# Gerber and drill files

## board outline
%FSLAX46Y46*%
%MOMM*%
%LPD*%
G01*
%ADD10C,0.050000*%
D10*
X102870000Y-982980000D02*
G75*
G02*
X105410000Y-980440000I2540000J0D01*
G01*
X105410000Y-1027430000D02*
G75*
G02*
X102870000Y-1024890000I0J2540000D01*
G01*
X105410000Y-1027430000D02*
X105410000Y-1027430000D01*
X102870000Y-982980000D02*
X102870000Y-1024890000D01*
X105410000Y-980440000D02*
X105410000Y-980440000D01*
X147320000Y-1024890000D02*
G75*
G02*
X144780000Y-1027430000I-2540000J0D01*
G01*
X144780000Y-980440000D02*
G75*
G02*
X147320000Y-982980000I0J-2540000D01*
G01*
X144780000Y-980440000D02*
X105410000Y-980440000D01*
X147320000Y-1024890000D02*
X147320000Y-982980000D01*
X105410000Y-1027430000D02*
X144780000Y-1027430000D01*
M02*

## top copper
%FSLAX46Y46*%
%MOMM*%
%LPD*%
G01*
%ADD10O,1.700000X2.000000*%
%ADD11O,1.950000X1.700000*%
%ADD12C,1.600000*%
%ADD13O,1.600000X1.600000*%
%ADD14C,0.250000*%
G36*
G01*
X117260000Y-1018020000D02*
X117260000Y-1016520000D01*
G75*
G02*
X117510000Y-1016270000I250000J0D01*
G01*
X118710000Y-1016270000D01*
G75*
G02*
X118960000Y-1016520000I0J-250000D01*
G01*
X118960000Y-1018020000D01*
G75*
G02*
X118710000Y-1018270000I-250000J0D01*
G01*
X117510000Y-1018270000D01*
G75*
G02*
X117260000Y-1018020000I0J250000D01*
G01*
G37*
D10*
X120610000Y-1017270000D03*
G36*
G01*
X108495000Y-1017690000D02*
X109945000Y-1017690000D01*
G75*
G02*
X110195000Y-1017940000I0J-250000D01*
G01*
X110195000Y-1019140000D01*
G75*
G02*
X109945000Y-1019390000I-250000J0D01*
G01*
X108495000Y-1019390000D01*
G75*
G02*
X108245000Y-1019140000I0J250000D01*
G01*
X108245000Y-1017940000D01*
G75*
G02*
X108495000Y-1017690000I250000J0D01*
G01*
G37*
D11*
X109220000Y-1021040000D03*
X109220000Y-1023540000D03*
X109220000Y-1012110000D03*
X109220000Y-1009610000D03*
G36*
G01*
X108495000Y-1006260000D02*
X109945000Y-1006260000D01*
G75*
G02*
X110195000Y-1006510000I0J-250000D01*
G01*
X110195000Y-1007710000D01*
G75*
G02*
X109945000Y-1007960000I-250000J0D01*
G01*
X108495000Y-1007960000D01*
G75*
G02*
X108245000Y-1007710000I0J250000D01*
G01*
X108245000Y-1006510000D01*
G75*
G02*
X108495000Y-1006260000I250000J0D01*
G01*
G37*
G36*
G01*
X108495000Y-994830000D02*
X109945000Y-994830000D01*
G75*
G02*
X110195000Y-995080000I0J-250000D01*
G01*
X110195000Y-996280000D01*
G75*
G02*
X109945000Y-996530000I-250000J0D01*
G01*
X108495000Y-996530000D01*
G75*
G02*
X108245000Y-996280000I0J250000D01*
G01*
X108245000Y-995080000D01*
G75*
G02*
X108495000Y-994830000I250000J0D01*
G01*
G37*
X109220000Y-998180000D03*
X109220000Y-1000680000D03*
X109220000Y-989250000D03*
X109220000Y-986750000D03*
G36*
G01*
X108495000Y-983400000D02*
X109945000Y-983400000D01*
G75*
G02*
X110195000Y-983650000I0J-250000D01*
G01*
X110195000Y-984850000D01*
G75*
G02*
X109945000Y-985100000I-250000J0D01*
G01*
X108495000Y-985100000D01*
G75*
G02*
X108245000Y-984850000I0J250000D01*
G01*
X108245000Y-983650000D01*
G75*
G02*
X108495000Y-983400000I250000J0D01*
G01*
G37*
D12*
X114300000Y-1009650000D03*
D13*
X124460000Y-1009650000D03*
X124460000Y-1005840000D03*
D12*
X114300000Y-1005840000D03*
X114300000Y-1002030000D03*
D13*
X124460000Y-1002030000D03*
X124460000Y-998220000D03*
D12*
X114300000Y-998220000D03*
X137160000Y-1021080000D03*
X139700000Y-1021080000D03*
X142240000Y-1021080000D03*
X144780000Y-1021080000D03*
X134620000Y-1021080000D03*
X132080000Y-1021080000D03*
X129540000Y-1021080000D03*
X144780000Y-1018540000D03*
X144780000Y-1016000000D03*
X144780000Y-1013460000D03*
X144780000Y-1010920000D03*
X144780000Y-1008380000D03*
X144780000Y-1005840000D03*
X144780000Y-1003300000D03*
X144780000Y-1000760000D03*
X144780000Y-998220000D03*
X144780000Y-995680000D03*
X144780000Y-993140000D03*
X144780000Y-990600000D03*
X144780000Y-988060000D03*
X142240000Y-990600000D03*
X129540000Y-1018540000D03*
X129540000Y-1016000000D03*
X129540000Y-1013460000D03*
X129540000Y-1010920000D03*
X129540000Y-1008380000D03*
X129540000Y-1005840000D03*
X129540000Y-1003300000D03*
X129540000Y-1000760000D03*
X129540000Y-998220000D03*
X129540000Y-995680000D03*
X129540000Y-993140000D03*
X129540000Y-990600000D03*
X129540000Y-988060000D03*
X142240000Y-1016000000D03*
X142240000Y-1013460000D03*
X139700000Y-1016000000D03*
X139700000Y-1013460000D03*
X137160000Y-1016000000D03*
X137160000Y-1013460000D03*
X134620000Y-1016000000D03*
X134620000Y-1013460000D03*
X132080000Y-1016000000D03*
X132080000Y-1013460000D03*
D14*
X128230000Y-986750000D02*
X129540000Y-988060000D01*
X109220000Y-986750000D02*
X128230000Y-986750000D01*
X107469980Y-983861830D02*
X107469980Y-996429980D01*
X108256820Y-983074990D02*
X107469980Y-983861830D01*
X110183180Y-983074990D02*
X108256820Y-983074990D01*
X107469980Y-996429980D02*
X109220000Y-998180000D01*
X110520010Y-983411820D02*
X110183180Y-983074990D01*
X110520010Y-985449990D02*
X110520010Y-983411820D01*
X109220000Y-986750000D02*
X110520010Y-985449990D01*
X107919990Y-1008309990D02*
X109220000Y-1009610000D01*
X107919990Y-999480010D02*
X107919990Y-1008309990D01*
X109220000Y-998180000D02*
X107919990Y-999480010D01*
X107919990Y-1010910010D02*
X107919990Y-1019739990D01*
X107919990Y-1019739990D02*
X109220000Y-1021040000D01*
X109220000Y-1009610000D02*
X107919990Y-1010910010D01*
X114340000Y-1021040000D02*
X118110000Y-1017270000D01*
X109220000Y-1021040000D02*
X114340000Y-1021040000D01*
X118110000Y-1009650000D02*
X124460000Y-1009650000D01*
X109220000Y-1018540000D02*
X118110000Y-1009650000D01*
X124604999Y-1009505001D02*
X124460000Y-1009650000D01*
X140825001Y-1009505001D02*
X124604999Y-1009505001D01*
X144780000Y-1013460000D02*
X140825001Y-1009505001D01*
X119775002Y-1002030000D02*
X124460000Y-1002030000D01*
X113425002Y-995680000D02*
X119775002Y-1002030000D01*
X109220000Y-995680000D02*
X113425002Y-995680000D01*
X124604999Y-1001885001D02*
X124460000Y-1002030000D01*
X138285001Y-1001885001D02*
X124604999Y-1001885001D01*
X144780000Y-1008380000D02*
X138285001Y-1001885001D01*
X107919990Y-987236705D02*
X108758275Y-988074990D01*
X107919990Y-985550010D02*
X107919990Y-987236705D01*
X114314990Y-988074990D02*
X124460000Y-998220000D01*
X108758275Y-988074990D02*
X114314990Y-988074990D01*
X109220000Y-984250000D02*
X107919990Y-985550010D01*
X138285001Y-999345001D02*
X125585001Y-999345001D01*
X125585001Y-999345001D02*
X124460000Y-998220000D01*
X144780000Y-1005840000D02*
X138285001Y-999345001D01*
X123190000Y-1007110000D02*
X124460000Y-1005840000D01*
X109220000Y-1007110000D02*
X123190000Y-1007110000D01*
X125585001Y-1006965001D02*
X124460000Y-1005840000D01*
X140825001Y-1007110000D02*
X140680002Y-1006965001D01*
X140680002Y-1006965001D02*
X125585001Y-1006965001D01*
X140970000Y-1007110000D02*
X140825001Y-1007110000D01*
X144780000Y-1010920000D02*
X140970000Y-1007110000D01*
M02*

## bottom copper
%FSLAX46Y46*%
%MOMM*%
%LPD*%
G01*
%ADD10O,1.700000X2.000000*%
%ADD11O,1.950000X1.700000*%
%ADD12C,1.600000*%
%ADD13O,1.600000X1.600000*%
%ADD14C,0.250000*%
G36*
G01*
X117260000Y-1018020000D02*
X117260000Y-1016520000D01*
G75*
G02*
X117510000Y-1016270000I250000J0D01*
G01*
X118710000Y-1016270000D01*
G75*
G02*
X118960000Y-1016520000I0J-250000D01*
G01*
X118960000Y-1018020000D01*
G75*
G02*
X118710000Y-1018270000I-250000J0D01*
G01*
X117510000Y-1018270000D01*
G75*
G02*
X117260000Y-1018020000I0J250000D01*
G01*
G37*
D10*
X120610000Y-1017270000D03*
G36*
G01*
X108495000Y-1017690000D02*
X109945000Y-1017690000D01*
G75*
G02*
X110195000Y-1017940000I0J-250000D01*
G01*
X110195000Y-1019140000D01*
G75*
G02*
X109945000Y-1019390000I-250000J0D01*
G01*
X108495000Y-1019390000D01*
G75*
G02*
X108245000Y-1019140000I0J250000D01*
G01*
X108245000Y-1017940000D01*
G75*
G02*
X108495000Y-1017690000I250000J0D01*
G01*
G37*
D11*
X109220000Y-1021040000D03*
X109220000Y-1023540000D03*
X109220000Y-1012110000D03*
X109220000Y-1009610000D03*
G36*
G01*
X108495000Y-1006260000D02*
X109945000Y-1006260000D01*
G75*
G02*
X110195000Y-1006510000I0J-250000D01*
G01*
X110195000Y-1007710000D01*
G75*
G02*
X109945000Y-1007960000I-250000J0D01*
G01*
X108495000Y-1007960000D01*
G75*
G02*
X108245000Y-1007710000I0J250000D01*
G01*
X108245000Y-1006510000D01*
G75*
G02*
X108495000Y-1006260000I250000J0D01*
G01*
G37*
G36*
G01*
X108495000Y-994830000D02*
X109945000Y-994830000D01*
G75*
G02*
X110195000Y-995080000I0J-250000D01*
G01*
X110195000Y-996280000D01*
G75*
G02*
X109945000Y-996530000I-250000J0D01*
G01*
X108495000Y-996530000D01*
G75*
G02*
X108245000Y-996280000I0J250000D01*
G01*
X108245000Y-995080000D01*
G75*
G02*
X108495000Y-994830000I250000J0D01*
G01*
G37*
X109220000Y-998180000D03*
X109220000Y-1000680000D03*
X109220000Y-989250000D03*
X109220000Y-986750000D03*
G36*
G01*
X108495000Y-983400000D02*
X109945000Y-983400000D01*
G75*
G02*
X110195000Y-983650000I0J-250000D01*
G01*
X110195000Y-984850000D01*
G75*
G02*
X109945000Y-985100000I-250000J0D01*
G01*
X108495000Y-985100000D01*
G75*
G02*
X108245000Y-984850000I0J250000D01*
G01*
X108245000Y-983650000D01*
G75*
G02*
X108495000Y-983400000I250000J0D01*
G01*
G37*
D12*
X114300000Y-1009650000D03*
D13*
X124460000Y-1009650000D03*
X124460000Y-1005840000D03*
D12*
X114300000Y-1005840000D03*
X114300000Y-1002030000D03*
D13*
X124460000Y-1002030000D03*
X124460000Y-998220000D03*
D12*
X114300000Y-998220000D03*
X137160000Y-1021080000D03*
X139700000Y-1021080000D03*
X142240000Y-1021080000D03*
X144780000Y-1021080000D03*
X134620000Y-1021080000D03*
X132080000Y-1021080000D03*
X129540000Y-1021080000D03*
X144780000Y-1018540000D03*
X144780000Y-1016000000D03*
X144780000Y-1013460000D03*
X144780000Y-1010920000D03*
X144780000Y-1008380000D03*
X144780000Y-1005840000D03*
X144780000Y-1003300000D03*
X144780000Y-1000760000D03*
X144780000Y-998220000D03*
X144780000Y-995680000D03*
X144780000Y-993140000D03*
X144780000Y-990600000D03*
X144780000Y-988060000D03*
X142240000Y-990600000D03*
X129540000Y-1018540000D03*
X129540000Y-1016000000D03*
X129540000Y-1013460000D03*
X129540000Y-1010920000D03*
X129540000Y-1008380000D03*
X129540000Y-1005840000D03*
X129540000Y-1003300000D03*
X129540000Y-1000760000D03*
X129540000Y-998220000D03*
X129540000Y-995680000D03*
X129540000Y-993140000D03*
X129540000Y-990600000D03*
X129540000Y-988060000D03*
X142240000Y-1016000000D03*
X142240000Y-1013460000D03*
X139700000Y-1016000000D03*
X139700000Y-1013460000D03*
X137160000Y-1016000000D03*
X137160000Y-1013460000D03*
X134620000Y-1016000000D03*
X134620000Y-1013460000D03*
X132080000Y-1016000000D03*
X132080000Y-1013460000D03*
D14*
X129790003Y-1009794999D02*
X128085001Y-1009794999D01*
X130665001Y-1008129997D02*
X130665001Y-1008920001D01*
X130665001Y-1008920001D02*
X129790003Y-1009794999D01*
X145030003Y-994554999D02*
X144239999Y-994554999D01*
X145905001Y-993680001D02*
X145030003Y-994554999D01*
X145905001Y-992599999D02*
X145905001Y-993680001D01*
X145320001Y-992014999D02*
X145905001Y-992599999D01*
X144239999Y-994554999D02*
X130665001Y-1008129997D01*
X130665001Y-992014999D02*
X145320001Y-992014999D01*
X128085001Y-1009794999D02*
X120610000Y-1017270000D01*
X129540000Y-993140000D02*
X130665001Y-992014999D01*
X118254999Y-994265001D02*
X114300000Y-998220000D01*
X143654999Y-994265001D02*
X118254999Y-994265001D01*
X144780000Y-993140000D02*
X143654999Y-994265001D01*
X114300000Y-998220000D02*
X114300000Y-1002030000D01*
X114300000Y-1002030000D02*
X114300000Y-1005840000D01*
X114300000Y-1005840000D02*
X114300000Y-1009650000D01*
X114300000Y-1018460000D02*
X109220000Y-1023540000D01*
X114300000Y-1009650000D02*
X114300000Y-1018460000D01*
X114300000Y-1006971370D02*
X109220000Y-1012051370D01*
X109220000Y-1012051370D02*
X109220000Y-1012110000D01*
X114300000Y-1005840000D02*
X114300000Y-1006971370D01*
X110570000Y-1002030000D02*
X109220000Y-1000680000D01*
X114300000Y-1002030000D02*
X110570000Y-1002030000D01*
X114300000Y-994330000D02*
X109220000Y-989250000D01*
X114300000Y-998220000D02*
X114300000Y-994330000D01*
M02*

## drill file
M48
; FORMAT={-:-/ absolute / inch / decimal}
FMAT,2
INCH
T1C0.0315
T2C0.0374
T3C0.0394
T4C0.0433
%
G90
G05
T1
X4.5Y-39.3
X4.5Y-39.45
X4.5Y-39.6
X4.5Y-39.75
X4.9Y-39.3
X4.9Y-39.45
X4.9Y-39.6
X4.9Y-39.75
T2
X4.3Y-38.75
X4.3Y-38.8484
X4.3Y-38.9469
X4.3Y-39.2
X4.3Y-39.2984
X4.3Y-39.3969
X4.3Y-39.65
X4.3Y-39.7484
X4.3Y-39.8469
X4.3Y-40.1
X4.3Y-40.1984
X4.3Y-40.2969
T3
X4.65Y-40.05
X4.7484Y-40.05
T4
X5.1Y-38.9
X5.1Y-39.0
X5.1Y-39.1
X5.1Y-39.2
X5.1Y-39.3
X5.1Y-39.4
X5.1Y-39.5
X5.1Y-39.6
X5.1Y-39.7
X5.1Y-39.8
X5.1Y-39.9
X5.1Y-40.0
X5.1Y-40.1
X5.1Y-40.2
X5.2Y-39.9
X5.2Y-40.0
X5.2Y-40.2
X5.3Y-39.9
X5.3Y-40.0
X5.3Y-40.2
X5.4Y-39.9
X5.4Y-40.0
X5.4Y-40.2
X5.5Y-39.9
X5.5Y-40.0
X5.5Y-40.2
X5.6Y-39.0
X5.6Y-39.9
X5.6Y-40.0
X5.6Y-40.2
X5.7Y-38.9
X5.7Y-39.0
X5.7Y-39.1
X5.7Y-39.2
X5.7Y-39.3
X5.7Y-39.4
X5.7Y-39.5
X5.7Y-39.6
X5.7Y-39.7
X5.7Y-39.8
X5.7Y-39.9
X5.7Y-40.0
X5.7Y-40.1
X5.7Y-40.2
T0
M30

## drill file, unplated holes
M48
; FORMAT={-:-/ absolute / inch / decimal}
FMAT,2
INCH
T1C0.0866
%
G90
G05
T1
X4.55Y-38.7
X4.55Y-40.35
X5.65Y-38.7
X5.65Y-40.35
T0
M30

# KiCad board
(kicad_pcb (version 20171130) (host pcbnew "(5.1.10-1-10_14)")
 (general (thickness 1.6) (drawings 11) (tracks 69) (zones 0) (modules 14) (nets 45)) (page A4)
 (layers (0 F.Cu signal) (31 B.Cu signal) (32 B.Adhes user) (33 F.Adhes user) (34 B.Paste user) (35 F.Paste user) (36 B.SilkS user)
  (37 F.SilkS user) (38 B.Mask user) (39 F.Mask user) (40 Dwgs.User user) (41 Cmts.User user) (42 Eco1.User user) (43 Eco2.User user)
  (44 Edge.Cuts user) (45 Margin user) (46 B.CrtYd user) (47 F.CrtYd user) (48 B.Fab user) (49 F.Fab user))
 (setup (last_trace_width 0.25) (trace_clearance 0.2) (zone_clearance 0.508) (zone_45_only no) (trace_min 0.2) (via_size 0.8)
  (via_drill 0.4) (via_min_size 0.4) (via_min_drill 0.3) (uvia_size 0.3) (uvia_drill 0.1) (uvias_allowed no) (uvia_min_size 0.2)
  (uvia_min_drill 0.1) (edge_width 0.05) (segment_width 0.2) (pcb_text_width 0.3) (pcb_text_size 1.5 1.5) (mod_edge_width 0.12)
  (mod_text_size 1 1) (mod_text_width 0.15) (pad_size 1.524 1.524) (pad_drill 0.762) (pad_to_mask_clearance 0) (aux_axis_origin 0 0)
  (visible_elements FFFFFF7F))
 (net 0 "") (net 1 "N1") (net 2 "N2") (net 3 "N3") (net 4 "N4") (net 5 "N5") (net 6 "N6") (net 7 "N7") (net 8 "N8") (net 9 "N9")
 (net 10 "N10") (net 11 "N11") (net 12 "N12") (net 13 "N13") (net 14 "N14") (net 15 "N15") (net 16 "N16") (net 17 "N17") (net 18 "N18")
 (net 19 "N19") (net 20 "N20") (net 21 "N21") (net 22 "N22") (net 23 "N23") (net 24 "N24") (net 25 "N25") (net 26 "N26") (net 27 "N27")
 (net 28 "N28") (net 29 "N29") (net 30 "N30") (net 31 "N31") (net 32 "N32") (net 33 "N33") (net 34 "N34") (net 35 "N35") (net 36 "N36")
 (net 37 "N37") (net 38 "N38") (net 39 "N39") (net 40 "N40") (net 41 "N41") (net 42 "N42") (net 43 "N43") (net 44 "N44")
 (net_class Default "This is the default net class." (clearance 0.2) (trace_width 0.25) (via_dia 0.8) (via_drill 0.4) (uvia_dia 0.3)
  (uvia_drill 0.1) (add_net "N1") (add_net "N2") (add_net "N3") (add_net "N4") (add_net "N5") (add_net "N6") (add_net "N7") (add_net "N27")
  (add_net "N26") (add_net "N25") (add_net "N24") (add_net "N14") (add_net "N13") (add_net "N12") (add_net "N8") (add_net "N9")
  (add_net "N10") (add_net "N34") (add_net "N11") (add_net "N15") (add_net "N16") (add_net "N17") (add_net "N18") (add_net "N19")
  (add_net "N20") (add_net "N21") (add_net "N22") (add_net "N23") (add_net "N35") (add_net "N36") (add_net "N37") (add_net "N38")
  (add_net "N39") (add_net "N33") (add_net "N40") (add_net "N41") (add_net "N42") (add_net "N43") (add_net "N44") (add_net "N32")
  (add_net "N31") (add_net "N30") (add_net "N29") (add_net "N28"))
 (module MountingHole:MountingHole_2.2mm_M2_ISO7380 (layer F.Cu) (at 115.57 1024.89)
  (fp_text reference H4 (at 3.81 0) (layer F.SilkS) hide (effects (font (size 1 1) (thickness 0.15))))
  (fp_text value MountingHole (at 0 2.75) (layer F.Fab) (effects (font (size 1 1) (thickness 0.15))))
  (pad 1 np_thru_hole circle (at 0 0) (size 2.2 2.2) (drill 2.2) (layers *.Cu *.Mask)))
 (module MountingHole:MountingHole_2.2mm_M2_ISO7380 (layer F.Cu) (at 143.51 1024.89)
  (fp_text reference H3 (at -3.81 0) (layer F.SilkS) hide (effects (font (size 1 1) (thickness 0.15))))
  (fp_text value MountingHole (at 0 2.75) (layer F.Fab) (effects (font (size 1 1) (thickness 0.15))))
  (pad 1 np_thru_hole circle (at 0 0) (size 2.2 2.2) (drill 2.2) (layers *.Cu *.Mask)))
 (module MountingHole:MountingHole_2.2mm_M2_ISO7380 (layer F.Cu) (at 143.51 982.98)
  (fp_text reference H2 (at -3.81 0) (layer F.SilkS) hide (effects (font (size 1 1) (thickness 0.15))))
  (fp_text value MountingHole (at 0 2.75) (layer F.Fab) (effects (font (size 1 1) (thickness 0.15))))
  (pad 1 np_thru_hole circle (at 0 0) (size 2.2 2.2) (drill 2.2) (layers *.Cu *.Mask)))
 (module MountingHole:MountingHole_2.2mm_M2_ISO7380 (layer F.Cu) (at 115.57 982.98)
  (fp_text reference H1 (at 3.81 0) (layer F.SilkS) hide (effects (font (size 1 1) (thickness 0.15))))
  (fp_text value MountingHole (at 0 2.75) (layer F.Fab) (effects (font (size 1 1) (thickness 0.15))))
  (pad 1 np_thru_hole circle (at 0 0) (size 2.2 2.2) (drill 2.2) (layers *.Cu *.Mask)))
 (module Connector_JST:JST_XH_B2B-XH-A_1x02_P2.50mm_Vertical (layer F.Cu) (at 118.11 1017.27)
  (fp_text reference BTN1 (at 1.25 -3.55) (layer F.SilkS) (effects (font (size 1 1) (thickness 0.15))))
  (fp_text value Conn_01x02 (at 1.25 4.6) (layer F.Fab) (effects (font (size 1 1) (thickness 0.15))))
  (pad 1 thru_hole roundrect (at 0 0) (size 1.7 2) (drill 1) (layers *.Cu *.Mask) (roundrect_rratio 0.1470588235294118) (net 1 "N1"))
  (pad 2 thru_hole oval (at 2.5 0) (size 1.7 2) (drill 1) (layers *.Cu *.Mask) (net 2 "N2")))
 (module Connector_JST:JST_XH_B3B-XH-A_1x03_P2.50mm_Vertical (layer F.Cu) (at 109.22 1018.54 270)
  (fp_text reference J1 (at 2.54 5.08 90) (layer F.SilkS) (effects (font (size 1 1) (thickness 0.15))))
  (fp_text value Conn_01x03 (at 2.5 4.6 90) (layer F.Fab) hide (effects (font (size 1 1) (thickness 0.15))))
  (pad 1 thru_hole roundrect (at 0 0 270) (size 1.7 1.95) (drill 0.95) (layers *.Cu *.Mask) (roundrect_rratio 0.1470588235294118)
   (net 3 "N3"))
  (pad 2 thru_hole oval (at 2.5 0 270) (size 1.7 1.95) (drill 0.95) (layers *.Cu *.Mask) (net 1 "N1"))
  (pad 3 thru_hole oval (at 5 0 270) (size 1.7 1.95) (drill 0.95) (layers *.Cu *.Mask) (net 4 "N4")))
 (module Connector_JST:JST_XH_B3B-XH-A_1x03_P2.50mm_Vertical (layer F.Cu) (at 109.22 1007.11 270)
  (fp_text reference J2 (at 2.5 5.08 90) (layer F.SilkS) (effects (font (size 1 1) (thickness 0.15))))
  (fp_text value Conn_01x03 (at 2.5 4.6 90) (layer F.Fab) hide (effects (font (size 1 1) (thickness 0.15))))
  (pad 3 thru_hole oval (at 5 0 270) (size 1.7 1.95) (drill 0.95) (layers *.Cu *.Mask) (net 4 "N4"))
  (pad 2 thru_hole oval (at 2.5 0 270) (size 1.7 1.95) (drill 0.95) (layers *.Cu *.Mask) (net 1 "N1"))
  (pad 1 thru_hole roundrect (at 0 0 270) (size 1.7 1.95) (drill 0.95) (layers *.Cu *.Mask) (roundrect_rratio 0.1470588235294118)
   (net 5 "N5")))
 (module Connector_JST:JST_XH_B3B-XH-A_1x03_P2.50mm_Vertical (layer F.Cu) (at 109.22 995.68 270)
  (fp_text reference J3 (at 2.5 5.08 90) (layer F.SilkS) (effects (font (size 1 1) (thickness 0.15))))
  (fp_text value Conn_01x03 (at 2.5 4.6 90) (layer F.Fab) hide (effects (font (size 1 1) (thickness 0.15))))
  (pad 1 thru_hole roundrect (at 0 0 270) (size 1.7 1.95) (drill 0.95) (layers *.Cu *.Mask) (roundrect_rratio 0.1470588235294118)
   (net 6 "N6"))
  (pad 2 thru_hole oval (at 2.5 0 270) (size 1.7 1.95) (drill 0.95) (layers *.Cu *.Mask) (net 1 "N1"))
  (pad 3 thru_hole oval (at 5 0 270) (size 1.7 1.95) (drill 0.95) (layers *.Cu *.Mask) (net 4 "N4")))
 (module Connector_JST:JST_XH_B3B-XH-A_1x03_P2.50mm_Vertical (layer F.Cu) (at 109.22 984.25 270)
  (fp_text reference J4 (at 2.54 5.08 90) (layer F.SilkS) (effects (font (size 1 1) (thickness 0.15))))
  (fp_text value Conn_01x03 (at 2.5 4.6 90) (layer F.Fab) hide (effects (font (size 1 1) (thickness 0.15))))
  (pad 3 thru_hole oval (at 5 0 270) (size 1.7 1.95) (drill 0.95) (layers *.Cu *.Mask) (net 4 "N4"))
  (pad 2 thru_hole oval (at 2.5 0 270) (size 1.7 1.95) (drill 0.95) (layers *.Cu *.Mask) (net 1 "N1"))
  (pad 1 thru_hole roundrect (at 0 0 270) (size 1.7 1.95) (drill 0.95) (layers *.Cu *.Mask) (roundrect_rratio 0.1470588235294118)
   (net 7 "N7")))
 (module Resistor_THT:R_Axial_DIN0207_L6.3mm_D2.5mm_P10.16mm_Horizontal (layer F.Cu) (at 114.3 1009.65)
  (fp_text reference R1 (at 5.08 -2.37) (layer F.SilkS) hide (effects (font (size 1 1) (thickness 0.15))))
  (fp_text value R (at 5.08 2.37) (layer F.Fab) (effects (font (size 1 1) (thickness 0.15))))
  (pad 1 thru_hole circle (at 0 0) (size 1.6 1.6) (drill 0.8) (layers *.Cu *.Mask) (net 4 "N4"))
  (pad 2 thru_hole oval (at 10.16 0) (size 1.6 1.6) (drill 0.8) (layers *.Cu *.Mask) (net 3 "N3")))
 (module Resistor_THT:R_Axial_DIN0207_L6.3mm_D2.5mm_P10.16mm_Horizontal (layer F.Cu) (at 114.3 1005.84)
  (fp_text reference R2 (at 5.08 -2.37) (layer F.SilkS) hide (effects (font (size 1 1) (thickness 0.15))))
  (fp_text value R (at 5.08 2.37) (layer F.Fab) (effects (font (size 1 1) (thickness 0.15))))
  (pad 2 thru_hole oval (at 10.16 0) (size 1.6 1.6) (drill 0.8) (layers *.Cu *.Mask) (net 5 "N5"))
  (pad 1 thru_hole circle (at 0 0) (size 1.6 1.6) (drill 0.8) (layers *.Cu *.Mask) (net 4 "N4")))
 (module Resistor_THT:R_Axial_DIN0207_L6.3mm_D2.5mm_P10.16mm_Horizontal (layer F.Cu) (at 114.3 1002.03)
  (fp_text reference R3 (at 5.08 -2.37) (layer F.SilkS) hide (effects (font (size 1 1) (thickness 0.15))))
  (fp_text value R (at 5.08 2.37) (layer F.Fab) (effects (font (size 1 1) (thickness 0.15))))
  (pad 1 thru_hole circle (at 0 0) (size 1.6 1.6) (drill 0.8) (layers *.Cu *.Mask) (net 4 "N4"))
  (pad 2 thru_hole oval (at 10.16 0) (size 1.6 1.6) (drill 0.8) (layers *.Cu *.Mask) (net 6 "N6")))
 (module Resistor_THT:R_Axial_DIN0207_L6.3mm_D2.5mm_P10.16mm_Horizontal (layer F.Cu) (at 114.3 998.22)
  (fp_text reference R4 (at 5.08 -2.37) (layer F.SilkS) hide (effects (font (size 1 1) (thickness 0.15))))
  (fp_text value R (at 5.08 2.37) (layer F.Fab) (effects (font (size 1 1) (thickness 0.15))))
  (pad 2 thru_hole oval (at 10.16 0) (size 1.6 1.6) (drill 0.8) (layers *.Cu *.Mask) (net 7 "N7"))
  (pad 1 thru_hole circle (at 0 0) (size 1.6 1.6) (drill 0.8) (layers *.Cu *.Mask) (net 4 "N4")))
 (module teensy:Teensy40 (layer F.Cu) (at 137.16 1004.57 270)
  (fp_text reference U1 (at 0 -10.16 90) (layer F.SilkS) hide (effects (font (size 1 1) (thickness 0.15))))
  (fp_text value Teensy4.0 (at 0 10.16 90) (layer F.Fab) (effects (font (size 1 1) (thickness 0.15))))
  (pad 17 thru_hole circle (at 16.51 0 270) (size 1.6 1.6) (drill 1.1) (layers *.Cu *.Mask) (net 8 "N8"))
  (pad 18 thru_hole circle (at 16.51 -2.54 270) (size 1.6 1.6) (drill 1.1) (layers *.Cu *.Mask) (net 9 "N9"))
  (pad 19 thru_hole circle (at 16.51 -5.08 270) (size 1.6 1.6) (drill 1.1) (layers *.Cu *.Mask) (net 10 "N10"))
  (pad 20 thru_hole circle (at 16.51 -7.62 270) (size 1.6 1.6) (drill 1.1) (layers *.Cu *.Mask) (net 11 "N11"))
  (pad 16 thru_hole circle (at 16.51 2.54 270) (size 1.6 1.6) (drill 1.1) (layers *.Cu *.Mask) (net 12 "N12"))
  (pad 15 thru_hole circle (at 16.51 5.08 270) (size 1.6 1.6) (drill 1.1) (layers *.Cu *.Mask) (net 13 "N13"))
  (pad 14 thru_hole circle (at 16.51 7.62 270) (size 1.6 1.6) (drill 1.1) (layers *.Cu *.Mask) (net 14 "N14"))
  (pad 21 thru_hole circle (at 13.97 -7.62 270) (size 1.6 1.6) (drill 1.1) (layers *.Cu *.Mask) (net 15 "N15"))
  (pad 22 thru_hole circle (at 11.43 -7.62 270) (size 1.6 1.6) (drill 1.1) (layers *.Cu *.Mask) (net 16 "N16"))
  (pad 23 thru_hole circle (at 8.89 -7.62 270) (size 1.6 1.6) (drill 1.1) (layers *.Cu *.Mask) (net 3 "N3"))
  (pad 24 thru_hole circle (at 6.35 -7.62 270) (size 1.6 1.6) (drill 1.1) (layers *.Cu *.Mask) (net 5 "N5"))
  (pad 25 thru_hole circle (at 3.81 -7.62 270) (size 1.6 1.6) (drill 1.1) (layers *.Cu *.Mask) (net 6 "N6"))
  (pad 26 thru_hole circle (at 1.27 -7.62 270) (size 1.6 1.6) (drill 1.1) (layers *.Cu *.Mask) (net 7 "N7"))
  (pad 27 thru_hole circle (at -1.27 -7.62 270) (size 1.6 1.6) (drill 1.1) (layers *.Cu *.Mask) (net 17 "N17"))
  (pad 28 thru_hole circle (at -3.81 -7.62 270) (size 1.6 1.6) (drill 1.1) (layers *.Cu *.Mask) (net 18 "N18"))
  (pad 29 thru_hole circle (at -6.35 -7.62 270) (size 1.6 1.6) (drill 1.1) (layers *.Cu *.Mask) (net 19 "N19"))
  (pad 30 thru_hole circle (at -8.89 -7.62 270) (size 1.6 1.6) (drill 1.1) (layers *.Cu *.Mask) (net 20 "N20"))
  (pad 31 thru_hole circle (at -11.43 -7.62 270) (size 1.6 1.6) (drill 1.1) (layers *.Cu *.Mask) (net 4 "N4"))
  (pad 32 thru_hole circle (at -13.97 -7.62 270) (size 1.6 1.6) (drill 1.1) (layers *.Cu *.Mask) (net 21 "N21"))
  (pad 33 thru_hole circle (at -16.51 -7.62 270) (size 1.6 1.6) (drill 1.1) (layers *.Cu *.Mask) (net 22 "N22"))
  (pad 34 thru_hole circle (at -13.97 -5.08 270) (size 1.6 1.6) (drill 1.1) (layers *.Cu *.Mask) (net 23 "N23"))
  (pad 13 thru_hole circle (at 13.97 7.62 270) (size 1.6 1.6) (drill 1.1) (layers *.Cu *.Mask) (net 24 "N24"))
  (pad 12 thru_hole circle (at 11.43 7.62 270) (size 1.6 1.6) (drill 1.1) (layers *.Cu *.Mask) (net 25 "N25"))
  (pad 11 thru_hole circle (at 8.89 7.62 270) (size 1.6 1.6) (drill 1.1) (layers *.Cu *.Mask) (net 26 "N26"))
  (pad 10 thru_hole circle (at 6.35 7.62 270) (size 1.6 1.6) (drill 1.1) (layers *.Cu *.Mask) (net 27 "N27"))
  (pad 9 thru_hole circle (at 3.81 7.62 270) (size 1.6 1.6) (drill 1.1) (layers *.Cu *.Mask) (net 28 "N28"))
  (pad 8 thru_hole circle (at 1.27 7.62 270) (size 1.6 1.6) (drill 1.1) (layers *.Cu *.Mask) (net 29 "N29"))
  (pad 7 thru_hole circle (at -1.27 7.62 270) (size 1.6 1.6) (drill 1.1) (layers *.Cu *.Mask) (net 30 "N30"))
  (pad 6 thru_hole circle (at -3.81 7.62 270) (size 1.6 1.6) (drill 1.1) (layers *.Cu *.Mask) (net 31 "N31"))
  (pad 5 thru_hole circle (at -6.35 7.62 270) (size 1.6 1.6) (drill 1.1) (layers *.Cu *.Mask) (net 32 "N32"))
  (pad 4 thru_hole circle (at -8.89 7.62 270) (size 1.6 1.6) (drill 1.1) (layers *.Cu *.Mask) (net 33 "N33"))
  (pad 3 thru_hole circle (at -11.43 7.62 270) (size 1.6 1.6) (drill 1.1) (layers *.Cu *.Mask) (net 2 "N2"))
  (pad 2 thru_hole circle (at -13.97 7.62 270) (size 1.6 1.6) (drill 1.1) (layers *.Cu *.Mask) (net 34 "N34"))
  (pad 1 thru_hole circle (at -16.51 7.62 270) (size 1.6 1.6) (drill 1.1) (layers *.Cu *.Mask) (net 1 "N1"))
  (pad 35 thru_hole circle (at 11.43 -5.08 270) (size 1.6 1.6) (drill 1.1) (layers *.Cu *.Mask) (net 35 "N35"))
  (pad 36 thru_hole circle (at 8.89 -5.08 270) (size 1.6 1.6) (drill 1.1) (layers *.Cu *.Mask) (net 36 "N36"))
  (pad 37 thru_hole circle (at 11.43 -2.54 270) (size 1.6 1.6) (drill 1.1) (layers *.Cu *.Mask) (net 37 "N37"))
  (pad 38 thru_hole circle (at 8.89 -2.54 270) (size 1.6 1.6) (drill 1.1) (layers *.Cu *.Mask) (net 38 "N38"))
  (pad 39 thru_hole circle (at 11.43 0 270) (size 1.6 1.6) (drill 1.1) (layers *.Cu *.Mask) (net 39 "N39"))
  (pad 40 thru_hole circle (at 8.89 0 270) (size 1.6 1.6) (drill 1.1) (layers *.Cu *.Mask) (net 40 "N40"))
  (pad 41 thru_hole circle (at 11.43 2.54 270) (size 1.6 1.6) (drill 1.1) (layers *.Cu *.Mask) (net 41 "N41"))
  (pad 42 thru_hole circle (at 8.89 2.54 270) (size 1.6 1.6) (drill 1.1) (layers *.Cu *.Mask) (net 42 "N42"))
  (pad 43 thru_hole circle (at 11.43 5.08 270) (size 1.6 1.6) (drill 1.1) (layers *.Cu *.Mask) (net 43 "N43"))
  (pad 44 thru_hole circle (at 8.89 5.08 270) (size 1.6 1.6) (drill 1.1) (layers *.Cu *.Mask) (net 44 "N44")))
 (gr_arc (start 105.41 982.98) (end 105.41 980.44) (angle -90) (layer Edge.Cuts) (width 0.05))
 (gr_arc (start 105.41 1024.89) (end 102.87 1024.89) (angle -90) (layer Edge.Cuts) (width 0.05))
 (gr_line (start 105.41 1027.43) (end 105.41 1027.43) (layer Edge.Cuts) (width 0.05))
 (gr_line (start 102.87 982.98) (end 102.87 1024.89) (layer Edge.Cuts) (width 0.05))
 (gr_line (start 105.41 980.44) (end 105.41 980.44) (layer Edge.Cuts) (width 0.05))
 (gr_arc (start 144.78 1024.89) (end 144.78 1027.43) (angle -90) (layer Edge.Cuts) (width 0.05))
 (gr_arc (start 144.78 982.98) (end 147.32 982.98) (angle -90) (layer Edge.Cuts) (width 0.05))
 (gr_line (start 144.78 980.44) (end 105.41 980.44) (layer Edge.Cuts) (width 0.05))
 (gr_line (start 147.32 1024.89) (end 147.32 982.98) (layer Edge.Cuts) (width 0.05))
 (gr_line (start 105.41 1027.43) (end 144.78 1027.43) (layer Edge.Cuts) (width 0.05))
 (segment (start 128.23 986.75) (end 129.54 988.06) (width 0.25) (layer F.Cu) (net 1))
 (segment (start 109.22 986.75) (end 128.23 986.75) (width 0.25) (layer F.Cu) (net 1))
 (segment (start 107.46998 983.86183) (end 107.46998 996.42998) (width 0.25) (layer F.Cu) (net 1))
 (segment (start 108.25682 983.07499) (end 107.46998 983.86183) (width 0.25) (layer F.Cu) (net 1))
 (segment (start 110.18318 983.07499) (end 108.25682 983.07499) (width 0.25) (layer F.Cu) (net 1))
 (segment (start 107.46998 996.42998) (end 109.22 998.18) (width 0.25) (layer F.Cu) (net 1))
 (segment (start 110.52001 983.41182) (end 110.18318 983.07499) (width 0.25) (layer F.Cu) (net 1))
 (segment (start 110.52001 985.44999) (end 110.52001 983.41182) (width 0.25) (layer F.Cu) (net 1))
 (segment (start 109.22 986.75) (end 110.52001 985.44999) (width 0.25) (layer F.Cu) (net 1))
 (segment (start 107.91999 1008.30999) (end 109.22 1009.61) (width 0.25) (layer F.Cu) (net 1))
 (segment (start 107.91999 999.48001) (end 107.91999 1008.30999) (width 0.25) (layer F.Cu) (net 1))
 (segment (start 109.22 998.18) (end 107.91999 999.48001) (width 0.25) (layer F.Cu) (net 1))
 (segment (start 107.91999 1010.91001) (end 107.91999 1019.73999) (width 0.25) (layer F.Cu) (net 1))
 (segment (start 107.91999 1019.73999) (end 109.22 1021.04) (width 0.25) (layer F.Cu) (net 1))
 (segment (start 109.22 1009.61) (end 107.91999 1010.91001) (width 0.25) (layer F.Cu) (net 1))
 (segment (start 114.34 1021.04) (end 118.11 1017.27) (width 0.25) (layer F.Cu) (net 1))
 (segment (start 109.22 1021.04) (end 114.34 1021.04) (width 0.25) (layer F.Cu) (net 1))
 (segment (start 129.790003 1009.794999) (end 128.085001 1009.794999) (width 0.25) (layer B.Cu) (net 2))
 (segment (start 130.665001 1008.129997) (end 130.665001 1008.920001) (width 0.25) (layer B.Cu) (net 2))
 (segment (start 130.665001 1008.920001) (end 129.790003 1009.794999) (width 0.25) (layer B.Cu) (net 2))
 (segment (start 145.030003 994.554999) (end 144.239999 994.554999) (width 0.25) (layer B.Cu) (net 2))
 (segment (start 145.905001 993.680001) (end 145.030003 994.554999) (width 0.25) (layer B.Cu) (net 2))
 (segment (start 145.905001 992.599999) (end 145.905001 993.680001) (width 0.25) (layer B.Cu) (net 2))
 (segment (start 145.320001 992.014999) (end 145.905001 992.599999) (width 0.25) (layer B.Cu) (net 2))
 (segment (start 144.239999 994.554999) (end 130.665001 1008.129997) (width 0.25) (layer B.Cu) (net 2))
 (segment (start 130.665001 992.014999) (end 145.320001 992.014999) (width 0.25) (layer B.Cu) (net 2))
 (segment (start 128.085001 1009.794999) (end 120.61 1017.27) (width 0.25) (layer B.Cu) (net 2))
 (segment (start 129.54 993.14) (end 130.665001 992.014999) (width 0.25) (layer B.Cu) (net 2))
 (segment (start 118.11 1009.65) (end 124.46 1009.65) (width 0.25) (layer F.Cu) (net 3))
 (segment (start 109.22 1018.54) (end 118.11 1009.65) (width 0.25) (layer F.Cu) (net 3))
 (segment (start 124.604999 1009.505001) (end 124.46 1009.65) (width 0.25) (layer F.Cu) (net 3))
 (segment (start 140.825001 1009.505001) (end 124.604999 1009.505001) (width 0.25) (layer F.Cu) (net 3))
 (segment (start 144.78 1013.46) (end 140.825001 1009.505001) (width 0.25) (layer F.Cu) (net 3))
 (segment (start 118.254999 994.265001) (end 114.3 998.22) (width 0.25) (layer B.Cu) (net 4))
 (segment (start 143.654999 994.265001) (end 118.254999 994.265001) (width 0.25) (layer B.Cu) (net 4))
 (segment (start 144.78 993.14) (end 143.654999 994.265001) (width 0.25) (layer B.Cu) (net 4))
 (segment (start 114.3 998.22) (end 114.3 1002.03) (width 0.25) (layer B.Cu) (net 4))
 (segment (start 114.3 1002.03) (end 114.3 1005.84) (width 0.25) (layer B.Cu) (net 4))
 (segment (start 114.3 1005.84) (end 114.3 1009.65) (width 0.25) (layer B.Cu) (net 4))
 (segment (start 114.3 1018.46) (end 109.22 1023.54) (width 0.25) (layer B.Cu) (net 4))
 (segment (start 114.3 1009.65) (end 114.3 1018.46) (width 0.25) (layer B.Cu) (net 4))
 (segment (start 114.3 1006.97137) (end 109.22 1012.05137) (width 0.25) (layer B.Cu) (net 4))
 (segment (start 109.22 1012.05137) (end 109.22 1012.11) (width 0.25) (layer B.Cu) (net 4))
 (segment (start 114.3 1005.84) (end 114.3 1006.97137) (width 0.25) (layer B.Cu) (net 4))
 (segment (start 110.57 1002.03) (end 109.22 1000.68) (width 0.25) (layer B.Cu) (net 4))
 (segment (start 114.3 1002.03) (end 110.57 1002.03) (width 0.25) (layer B.Cu) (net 4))
 (segment (start 114.3 994.33) (end 109.22 989.25) (width 0.25) (layer B.Cu) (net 4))
 (segment (start 114.3 998.22) (end 114.3 994.33) (width 0.25) (layer B.Cu) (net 4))
 (segment (start 119.775002 1002.03) (end 124.46 1002.03) (width 0.25) (layer F.Cu) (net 6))
 (segment (start 113.425002 995.68) (end 119.775002 1002.03) (width 0.25) (layer F.Cu) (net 6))
 (segment (start 109.22 995.68) (end 113.425002 995.68) (width 0.25) (layer F.Cu) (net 6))
 (segment (start 124.604999 1001.885001) (end 124.46 1002.03) (width 0.25) (layer F.Cu) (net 6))
 (segment (start 138.285001 1001.885001) (end 124.604999 1001.885001) (width 0.25) (layer F.Cu) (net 6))
 (segment (start 144.78 1008.38) (end 138.285001 1001.885001) (width 0.25) (layer F.Cu) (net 6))
 (segment (start 107.91999 987.236705) (end 108.758275 988.07499) (width 0.25) (layer F.Cu) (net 7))
 (segment (start 107.91999 985.55001) (end 107.91999 987.236705) (width 0.25) (layer F.Cu) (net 7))
 (segment (start 114.31499 988.07499) (end 124.46 998.22) (width 0.25) (layer F.Cu) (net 7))
 (segment (start 108.758275 988.07499) (end 114.31499 988.07499) (width 0.25) (layer F.Cu) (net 7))
 (segment (start 109.22 984.25) (end 107.91999 985.55001) (width 0.25) (layer F.Cu) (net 7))
 (segment (start 138.285001 999.345001) (end 125.585001 999.345001) (width 0.25) (layer F.Cu) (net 7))
 (segment (start 125.585001 999.345001) (end 124.46 998.22) (width 0.25) (layer F.Cu) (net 7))
 (segment (start 144.78 1005.84) (end 138.285001 999.345001) (width 0.25) (layer F.Cu) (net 7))
 (segment (start 123.19 1007.11) (end 124.46 1005.84) (width 0.25) (layer F.Cu) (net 5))
 (segment (start 109.22 1007.11) (end 123.19 1007.11) (width 0.25) (layer F.Cu) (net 5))
 (segment (start 125.585001 1006.965001) (end 124.46 1005.84) (width 0.25) (layer F.Cu) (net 5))
 (segment (start 140.825001 1007.11) (end 140.680002 1006.965001) (width 0.25) (layer F.Cu) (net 5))
 (segment (start 140.680002 1006.965001) (end 125.585001 1006.965001) (width 0.25) (layer F.Cu) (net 5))
 (segment (start 140.97 1007.11) (end 140.825001 1007.11) (width 0.25) (layer F.Cu) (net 5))
 (segment (start 144.78 1010.92) (end 140.97 1007.11) (width 0.25) (layer F.Cu) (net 5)))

